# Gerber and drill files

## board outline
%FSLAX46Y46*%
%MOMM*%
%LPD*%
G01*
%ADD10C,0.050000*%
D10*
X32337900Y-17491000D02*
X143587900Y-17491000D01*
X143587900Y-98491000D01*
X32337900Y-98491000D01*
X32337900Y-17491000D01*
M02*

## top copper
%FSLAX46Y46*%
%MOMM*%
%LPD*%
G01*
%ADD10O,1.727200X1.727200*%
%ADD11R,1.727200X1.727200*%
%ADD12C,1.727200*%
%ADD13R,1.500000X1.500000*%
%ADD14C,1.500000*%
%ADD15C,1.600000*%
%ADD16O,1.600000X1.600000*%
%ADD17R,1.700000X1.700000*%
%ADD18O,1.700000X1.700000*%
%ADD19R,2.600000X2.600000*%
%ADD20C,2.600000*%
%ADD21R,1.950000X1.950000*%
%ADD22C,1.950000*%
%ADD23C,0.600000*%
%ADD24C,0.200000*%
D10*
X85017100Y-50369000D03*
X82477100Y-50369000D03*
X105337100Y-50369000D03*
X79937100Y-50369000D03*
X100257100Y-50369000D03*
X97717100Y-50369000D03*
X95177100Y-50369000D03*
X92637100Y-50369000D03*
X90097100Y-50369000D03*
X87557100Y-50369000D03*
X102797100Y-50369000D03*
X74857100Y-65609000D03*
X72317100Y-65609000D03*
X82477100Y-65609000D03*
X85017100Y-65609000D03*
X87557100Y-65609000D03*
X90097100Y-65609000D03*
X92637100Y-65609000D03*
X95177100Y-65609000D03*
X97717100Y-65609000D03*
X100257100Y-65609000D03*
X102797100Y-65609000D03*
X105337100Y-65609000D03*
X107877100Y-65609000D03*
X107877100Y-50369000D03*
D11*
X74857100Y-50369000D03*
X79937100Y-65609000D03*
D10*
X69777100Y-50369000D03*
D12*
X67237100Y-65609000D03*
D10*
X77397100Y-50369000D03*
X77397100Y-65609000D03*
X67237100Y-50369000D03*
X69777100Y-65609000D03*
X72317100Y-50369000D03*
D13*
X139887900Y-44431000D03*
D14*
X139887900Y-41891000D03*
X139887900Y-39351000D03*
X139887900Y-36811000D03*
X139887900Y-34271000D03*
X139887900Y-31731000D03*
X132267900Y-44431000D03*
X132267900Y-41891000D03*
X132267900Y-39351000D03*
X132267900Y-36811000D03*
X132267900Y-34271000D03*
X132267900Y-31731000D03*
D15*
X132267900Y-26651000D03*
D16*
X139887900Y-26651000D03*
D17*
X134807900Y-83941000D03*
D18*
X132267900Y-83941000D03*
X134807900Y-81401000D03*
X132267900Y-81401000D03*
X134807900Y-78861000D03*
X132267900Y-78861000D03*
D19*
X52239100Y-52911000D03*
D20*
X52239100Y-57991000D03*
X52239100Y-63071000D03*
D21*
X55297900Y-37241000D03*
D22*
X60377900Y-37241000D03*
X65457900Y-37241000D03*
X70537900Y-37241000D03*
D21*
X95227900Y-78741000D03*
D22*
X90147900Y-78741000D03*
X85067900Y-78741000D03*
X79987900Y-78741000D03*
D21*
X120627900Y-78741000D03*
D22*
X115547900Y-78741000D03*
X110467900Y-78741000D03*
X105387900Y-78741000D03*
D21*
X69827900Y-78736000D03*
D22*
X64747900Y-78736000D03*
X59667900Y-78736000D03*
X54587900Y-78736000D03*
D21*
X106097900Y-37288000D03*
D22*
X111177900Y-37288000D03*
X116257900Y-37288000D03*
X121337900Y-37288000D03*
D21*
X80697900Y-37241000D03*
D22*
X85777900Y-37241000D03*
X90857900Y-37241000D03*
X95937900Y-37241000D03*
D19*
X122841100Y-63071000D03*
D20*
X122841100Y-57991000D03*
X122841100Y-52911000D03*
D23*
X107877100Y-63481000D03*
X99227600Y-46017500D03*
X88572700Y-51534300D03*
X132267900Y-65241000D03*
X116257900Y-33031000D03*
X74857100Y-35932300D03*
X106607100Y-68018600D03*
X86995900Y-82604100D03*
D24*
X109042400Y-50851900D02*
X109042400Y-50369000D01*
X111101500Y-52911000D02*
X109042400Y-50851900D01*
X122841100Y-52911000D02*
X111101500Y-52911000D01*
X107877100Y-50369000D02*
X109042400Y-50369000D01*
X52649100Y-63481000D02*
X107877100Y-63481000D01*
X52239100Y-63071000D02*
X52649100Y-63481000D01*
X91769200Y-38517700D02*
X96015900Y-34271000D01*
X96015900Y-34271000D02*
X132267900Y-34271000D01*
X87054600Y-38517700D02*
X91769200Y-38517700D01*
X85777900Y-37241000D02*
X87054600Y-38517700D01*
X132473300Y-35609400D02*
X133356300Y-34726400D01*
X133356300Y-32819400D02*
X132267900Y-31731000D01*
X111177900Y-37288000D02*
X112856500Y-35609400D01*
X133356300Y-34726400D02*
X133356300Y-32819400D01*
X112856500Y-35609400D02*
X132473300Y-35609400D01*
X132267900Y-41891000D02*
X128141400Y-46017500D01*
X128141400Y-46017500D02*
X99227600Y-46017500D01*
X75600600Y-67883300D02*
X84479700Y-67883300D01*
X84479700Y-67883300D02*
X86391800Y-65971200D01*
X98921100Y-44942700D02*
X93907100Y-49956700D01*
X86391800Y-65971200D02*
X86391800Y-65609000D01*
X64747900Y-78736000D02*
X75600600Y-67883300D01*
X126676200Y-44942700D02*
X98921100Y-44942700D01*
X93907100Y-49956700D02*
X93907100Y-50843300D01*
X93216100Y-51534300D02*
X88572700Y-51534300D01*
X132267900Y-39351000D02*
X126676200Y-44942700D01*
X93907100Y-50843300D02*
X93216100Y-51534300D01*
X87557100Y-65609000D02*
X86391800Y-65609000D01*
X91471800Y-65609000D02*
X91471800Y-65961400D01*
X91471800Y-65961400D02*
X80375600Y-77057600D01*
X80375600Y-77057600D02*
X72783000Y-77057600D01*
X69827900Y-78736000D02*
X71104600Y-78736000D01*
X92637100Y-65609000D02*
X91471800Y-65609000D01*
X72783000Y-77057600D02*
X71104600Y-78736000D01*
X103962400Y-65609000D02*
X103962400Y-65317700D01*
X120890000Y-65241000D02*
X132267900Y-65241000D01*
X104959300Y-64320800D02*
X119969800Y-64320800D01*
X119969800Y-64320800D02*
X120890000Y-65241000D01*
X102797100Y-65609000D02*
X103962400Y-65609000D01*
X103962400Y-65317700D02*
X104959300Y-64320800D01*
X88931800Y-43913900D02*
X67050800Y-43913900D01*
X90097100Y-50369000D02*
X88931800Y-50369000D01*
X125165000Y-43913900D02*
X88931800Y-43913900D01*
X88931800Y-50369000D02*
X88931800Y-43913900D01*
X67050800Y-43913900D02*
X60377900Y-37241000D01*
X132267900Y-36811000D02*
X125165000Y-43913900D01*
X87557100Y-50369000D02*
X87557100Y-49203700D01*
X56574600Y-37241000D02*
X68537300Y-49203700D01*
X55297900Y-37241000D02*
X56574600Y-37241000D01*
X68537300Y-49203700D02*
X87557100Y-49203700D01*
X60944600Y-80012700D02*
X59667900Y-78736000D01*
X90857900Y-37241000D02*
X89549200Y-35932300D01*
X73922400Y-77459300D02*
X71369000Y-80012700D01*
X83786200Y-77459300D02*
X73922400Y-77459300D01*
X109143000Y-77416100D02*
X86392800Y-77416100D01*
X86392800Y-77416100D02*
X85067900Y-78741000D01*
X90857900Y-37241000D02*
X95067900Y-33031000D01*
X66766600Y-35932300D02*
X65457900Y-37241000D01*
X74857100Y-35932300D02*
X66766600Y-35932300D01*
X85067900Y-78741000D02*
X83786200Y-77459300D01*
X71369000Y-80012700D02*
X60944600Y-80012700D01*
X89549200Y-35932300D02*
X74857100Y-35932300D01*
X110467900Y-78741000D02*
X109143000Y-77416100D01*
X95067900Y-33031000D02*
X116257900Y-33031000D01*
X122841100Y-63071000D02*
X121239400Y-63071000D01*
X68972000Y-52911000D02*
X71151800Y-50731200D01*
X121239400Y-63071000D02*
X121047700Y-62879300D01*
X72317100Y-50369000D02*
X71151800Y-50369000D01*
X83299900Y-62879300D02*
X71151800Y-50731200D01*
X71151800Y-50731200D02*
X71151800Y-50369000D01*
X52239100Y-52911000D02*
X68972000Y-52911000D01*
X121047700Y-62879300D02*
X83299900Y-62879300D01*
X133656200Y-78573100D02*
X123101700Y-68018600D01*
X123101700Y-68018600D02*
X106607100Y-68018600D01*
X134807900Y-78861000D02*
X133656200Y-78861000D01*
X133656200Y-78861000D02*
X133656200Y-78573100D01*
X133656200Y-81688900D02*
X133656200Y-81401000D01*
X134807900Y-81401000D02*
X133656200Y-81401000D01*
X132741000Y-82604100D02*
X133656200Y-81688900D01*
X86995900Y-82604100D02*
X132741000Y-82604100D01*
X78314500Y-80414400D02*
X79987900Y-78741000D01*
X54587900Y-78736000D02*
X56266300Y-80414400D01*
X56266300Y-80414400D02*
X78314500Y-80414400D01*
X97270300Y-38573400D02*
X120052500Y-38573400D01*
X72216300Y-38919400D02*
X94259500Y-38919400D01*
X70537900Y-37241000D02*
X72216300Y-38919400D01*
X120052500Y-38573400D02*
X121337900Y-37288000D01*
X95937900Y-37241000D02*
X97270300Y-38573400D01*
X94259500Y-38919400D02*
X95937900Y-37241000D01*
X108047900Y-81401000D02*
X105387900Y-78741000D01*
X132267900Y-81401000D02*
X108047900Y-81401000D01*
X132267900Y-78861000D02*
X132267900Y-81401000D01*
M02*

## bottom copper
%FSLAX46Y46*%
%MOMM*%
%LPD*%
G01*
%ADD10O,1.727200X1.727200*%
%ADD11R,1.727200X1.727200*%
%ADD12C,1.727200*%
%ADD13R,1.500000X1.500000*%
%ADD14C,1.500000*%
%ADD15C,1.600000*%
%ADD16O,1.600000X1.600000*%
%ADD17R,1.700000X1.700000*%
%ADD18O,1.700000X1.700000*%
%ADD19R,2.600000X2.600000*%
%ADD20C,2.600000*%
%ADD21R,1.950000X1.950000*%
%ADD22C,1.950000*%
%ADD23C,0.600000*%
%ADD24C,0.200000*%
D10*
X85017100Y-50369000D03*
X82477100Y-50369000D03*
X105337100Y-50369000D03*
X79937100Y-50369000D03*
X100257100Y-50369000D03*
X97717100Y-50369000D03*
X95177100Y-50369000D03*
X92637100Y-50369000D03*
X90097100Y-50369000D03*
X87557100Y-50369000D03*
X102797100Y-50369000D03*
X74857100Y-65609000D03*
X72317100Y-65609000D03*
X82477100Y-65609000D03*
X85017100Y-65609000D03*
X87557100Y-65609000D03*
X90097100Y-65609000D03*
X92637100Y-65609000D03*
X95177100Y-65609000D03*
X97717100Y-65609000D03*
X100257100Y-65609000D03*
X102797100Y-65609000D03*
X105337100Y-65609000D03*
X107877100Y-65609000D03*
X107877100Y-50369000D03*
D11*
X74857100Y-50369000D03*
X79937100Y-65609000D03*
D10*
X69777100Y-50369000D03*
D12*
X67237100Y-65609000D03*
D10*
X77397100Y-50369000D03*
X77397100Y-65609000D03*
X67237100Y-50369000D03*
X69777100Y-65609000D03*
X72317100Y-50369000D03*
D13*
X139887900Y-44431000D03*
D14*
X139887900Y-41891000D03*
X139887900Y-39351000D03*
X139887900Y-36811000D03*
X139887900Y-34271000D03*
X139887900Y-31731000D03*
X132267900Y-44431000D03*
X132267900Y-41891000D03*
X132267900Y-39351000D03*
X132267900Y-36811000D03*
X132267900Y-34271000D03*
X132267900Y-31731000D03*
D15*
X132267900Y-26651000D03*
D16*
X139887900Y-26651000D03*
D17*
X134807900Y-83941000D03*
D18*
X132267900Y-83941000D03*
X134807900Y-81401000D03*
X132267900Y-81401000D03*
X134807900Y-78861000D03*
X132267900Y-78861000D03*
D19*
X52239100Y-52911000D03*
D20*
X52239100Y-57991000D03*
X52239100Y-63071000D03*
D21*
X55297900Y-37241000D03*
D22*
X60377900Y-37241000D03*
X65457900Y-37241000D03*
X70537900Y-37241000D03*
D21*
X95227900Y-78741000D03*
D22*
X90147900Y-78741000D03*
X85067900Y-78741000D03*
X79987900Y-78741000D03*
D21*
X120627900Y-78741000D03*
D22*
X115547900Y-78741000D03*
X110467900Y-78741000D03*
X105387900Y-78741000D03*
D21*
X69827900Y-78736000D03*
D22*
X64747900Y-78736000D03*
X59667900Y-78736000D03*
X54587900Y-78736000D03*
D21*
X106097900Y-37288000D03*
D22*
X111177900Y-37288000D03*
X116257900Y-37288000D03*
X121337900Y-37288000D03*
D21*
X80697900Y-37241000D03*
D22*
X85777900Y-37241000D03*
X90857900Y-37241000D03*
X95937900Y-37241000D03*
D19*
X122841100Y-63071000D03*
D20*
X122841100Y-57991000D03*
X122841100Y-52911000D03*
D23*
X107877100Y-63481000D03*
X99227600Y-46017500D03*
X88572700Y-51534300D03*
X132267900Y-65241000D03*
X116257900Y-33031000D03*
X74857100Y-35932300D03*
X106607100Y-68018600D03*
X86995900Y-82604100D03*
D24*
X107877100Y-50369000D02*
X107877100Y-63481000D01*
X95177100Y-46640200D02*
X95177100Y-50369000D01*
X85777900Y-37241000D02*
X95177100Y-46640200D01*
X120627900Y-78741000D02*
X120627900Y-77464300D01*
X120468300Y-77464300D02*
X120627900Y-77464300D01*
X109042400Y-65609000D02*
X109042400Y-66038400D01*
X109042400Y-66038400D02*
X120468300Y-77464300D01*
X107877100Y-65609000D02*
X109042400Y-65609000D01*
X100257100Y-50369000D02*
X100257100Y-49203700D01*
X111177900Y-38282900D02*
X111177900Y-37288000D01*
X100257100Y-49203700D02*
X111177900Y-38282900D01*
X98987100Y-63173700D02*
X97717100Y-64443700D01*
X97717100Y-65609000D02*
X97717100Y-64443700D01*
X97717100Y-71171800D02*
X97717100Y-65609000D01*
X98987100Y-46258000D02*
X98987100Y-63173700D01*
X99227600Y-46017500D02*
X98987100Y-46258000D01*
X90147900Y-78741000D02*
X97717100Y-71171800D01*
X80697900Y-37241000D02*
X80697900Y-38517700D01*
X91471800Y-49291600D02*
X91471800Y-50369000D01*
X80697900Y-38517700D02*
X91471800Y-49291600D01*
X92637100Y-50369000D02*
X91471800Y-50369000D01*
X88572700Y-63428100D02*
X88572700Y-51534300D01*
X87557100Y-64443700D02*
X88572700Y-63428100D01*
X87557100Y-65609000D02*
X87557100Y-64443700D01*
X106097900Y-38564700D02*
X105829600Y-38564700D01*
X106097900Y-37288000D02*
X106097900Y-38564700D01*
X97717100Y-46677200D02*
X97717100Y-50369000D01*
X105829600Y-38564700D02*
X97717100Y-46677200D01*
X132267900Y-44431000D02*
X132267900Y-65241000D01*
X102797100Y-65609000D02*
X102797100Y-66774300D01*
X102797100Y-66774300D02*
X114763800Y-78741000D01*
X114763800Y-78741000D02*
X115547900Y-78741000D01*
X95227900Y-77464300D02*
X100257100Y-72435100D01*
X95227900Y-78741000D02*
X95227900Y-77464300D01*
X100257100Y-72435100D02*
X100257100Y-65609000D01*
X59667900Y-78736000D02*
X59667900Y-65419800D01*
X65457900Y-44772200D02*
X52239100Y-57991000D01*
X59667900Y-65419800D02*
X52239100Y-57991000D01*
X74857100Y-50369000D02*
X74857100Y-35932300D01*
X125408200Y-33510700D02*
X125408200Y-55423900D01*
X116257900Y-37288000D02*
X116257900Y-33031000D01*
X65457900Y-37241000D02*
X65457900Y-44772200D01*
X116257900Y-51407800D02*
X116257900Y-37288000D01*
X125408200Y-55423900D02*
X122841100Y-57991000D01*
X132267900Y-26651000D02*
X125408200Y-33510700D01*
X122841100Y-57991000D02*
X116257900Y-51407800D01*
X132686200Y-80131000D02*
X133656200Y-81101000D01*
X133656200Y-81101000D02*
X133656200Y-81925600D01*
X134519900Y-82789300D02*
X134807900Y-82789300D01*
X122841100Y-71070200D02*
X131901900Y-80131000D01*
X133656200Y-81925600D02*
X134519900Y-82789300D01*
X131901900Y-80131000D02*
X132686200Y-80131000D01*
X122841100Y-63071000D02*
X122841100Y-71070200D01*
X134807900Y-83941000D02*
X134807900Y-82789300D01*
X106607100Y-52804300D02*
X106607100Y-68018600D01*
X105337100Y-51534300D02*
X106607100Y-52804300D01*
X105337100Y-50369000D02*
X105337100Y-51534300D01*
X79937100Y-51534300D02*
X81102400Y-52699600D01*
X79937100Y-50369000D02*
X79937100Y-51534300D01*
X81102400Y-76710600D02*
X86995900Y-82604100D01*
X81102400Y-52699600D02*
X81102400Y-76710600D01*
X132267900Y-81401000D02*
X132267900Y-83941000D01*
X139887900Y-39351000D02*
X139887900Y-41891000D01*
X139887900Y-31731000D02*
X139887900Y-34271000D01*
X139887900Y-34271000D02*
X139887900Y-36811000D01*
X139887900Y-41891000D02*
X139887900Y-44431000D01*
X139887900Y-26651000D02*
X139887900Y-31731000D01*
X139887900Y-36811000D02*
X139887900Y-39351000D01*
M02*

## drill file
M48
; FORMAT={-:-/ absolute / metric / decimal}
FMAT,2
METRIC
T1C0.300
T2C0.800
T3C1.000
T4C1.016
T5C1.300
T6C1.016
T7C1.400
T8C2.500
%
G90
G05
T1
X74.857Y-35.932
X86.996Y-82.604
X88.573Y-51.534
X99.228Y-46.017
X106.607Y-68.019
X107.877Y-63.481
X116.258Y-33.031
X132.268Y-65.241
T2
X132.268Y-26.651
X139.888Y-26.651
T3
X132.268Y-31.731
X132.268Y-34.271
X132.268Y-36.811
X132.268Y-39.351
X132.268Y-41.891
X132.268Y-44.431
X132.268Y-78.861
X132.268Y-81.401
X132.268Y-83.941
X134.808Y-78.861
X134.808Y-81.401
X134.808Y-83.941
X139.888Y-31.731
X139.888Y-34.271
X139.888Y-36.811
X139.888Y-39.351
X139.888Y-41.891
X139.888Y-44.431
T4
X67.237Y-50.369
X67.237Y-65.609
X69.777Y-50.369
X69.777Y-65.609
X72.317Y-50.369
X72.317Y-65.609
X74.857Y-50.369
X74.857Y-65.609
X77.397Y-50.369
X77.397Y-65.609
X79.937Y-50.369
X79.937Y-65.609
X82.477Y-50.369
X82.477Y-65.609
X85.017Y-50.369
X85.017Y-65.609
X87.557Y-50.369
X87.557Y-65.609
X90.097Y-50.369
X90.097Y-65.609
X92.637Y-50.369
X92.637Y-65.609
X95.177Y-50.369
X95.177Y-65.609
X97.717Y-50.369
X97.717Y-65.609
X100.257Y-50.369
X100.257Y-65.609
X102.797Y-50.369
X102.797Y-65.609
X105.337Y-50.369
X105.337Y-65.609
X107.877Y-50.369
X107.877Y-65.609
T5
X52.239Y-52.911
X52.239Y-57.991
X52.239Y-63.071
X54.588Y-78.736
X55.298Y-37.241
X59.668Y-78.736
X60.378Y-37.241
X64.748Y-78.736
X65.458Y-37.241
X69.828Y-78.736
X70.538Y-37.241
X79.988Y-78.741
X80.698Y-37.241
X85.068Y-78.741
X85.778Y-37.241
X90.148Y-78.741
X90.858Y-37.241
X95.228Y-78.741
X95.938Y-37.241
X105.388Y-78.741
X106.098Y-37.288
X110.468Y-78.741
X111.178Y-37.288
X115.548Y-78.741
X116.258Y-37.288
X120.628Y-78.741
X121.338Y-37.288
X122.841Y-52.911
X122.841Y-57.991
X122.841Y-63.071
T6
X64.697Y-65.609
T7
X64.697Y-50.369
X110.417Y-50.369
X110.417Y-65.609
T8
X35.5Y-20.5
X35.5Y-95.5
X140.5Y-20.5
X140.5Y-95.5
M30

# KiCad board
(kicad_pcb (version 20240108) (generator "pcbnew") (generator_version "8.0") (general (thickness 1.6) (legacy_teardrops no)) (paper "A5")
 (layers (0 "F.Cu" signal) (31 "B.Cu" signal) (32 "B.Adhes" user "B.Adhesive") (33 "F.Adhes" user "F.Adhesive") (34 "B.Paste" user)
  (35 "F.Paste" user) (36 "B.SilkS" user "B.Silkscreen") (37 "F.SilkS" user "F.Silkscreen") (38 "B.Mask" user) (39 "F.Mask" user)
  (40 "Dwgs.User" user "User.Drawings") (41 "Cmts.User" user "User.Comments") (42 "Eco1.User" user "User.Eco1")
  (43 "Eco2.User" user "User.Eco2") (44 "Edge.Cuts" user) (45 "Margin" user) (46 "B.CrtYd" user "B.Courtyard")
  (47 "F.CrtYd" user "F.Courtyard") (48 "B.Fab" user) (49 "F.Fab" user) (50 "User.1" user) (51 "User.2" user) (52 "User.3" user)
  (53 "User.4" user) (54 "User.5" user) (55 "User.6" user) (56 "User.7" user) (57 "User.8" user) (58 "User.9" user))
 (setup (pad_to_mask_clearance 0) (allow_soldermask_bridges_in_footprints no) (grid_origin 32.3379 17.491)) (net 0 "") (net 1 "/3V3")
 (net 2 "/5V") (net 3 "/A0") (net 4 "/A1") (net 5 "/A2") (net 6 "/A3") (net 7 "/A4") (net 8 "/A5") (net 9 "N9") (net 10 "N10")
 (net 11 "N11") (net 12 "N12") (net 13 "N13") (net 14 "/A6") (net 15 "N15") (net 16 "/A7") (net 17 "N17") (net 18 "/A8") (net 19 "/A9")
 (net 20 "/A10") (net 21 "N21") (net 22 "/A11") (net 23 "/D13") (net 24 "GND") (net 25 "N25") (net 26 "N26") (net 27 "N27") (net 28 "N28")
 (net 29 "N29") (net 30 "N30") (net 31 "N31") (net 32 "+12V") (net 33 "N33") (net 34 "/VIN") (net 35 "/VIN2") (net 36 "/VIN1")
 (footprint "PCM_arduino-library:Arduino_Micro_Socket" (layer "F.Cu") (at 111.7971 48.989 180)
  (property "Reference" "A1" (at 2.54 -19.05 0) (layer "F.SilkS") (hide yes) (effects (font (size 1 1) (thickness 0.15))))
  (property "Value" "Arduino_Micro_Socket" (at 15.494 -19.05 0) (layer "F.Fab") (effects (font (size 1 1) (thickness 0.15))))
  (pad "" np_thru_hole circle (at 1.38 -16.62 180) (size 1.4 1.4) (drill 1.4) (layers "F&B.Cu" "*.Mask"))
  (pad "" np_thru_hole circle (at 1.38 -1.38 180) (size 1.4 1.4) (drill 1.4) (layers "F&B.Cu" "*.Mask"))
  (pad "" thru_hole oval (at 26.78 -1.38 180) (size 1.7272 1.7272) (drill 1.016) (layers "*.Cu" "*.Mask") (remove_unused_layers no))
  (pad "" thru_hole oval (at 29.32 -1.38 180) (size 1.7272 1.7272) (drill 1.016) (layers "*.Cu" "*.Mask") (remove_unused_layers no))
  (pad "" np_thru_hole circle (at 47.1 -16.62 180) (size 1.016 1.016) (drill 1.016) (layers "*.Cu" "*.Mask"))
  (pad "" np_thru_hole circle (at 47.1 -1.38 180) (size 1.4 1.4) (drill 1.4) (layers "F&B.Cu" "*.Mask"))
  (pad "3V3" thru_hole oval (at 6.46 -1.38 180) (size 1.7272 1.7272) (drill 1.016) (layers "*.Cu" "*.Mask") (remove_unused_layers no)
   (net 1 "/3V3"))
  (pad "5V" thru_hole oval (at 31.86 -1.38 180) (size 1.7272 1.7272) (drill 1.016) (layers "*.Cu" "*.Mask") (remove_unused_layers no)
   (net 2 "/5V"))
  (pad "A0" thru_hole oval (at 11.54 -1.38 180) (size 1.7272 1.7272) (drill 1.016) (layers "*.Cu" "*.Mask") (remove_unused_layers no)
   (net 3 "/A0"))
  (pad "A1" thru_hole oval (at 14.08 -1.38 180) (size 1.7272 1.7272) (drill 1.016) (layers "*.Cu" "*.Mask") (remove_unused_layers no)
   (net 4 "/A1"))
  (pad "A2" thru_hole oval (at 16.62 -1.38 180) (size 1.7272 1.7272) (drill 1.016) (layers "*.Cu" "*.Mask") (remove_unused_layers no)
   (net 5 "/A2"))
  (pad "A3" thru_hole oval (at 19.16 -1.38 180) (size 1.7272 1.7272) (drill 1.016) (layers "*.Cu" "*.Mask") (remove_unused_layers no)
   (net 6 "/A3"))
  (pad "A4" thru_hole oval (at 21.7 -1.38 180) (size 1.7272 1.7272) (drill 1.016) (layers "*.Cu" "*.Mask") (remove_unused_layers no)
   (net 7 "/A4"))
  (pad "A5" thru_hole oval (at 24.24 -1.38 180) (size 1.7272 1.7272) (drill 1.016) (layers "*.Cu" "*.Mask") (remove_unused_layers no)
   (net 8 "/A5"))
  (pad "AREF" thru_hole oval (at 9 -1.38 180) (size 1.7272 1.7272) (drill 1.016) (layers "*.Cu" "*.Mask") (remove_unused_layers no)
   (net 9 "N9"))
  (pad "D0" thru_hole oval (at 36.94 -16.62 180) (size 1.7272 1.7272) (drill 1.016) (layers "*.Cu" "*.Mask") (remove_unused_layers no)
   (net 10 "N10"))
  (pad "D1" thru_hole oval (at 39.48 -16.62 180) (size 1.7272 1.7272) (drill 1.016) (layers "*.Cu" "*.Mask") (remove_unused_layers no)
   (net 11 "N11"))
  (pad "D2" thru_hole oval (at 29.32 -16.62 180) (size 1.7272 1.7272) (drill 1.016) (layers "*.Cu" "*.Mask") (remove_unused_layers no)
   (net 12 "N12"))
  (pad "D3" thru_hole oval (at 26.78 -16.62 180) (size 1.7272 1.7272) (drill 1.016) (layers "*.Cu" "*.Mask") (remove_unused_layers no)
   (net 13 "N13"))
  (pad "D4" thru_hole oval (at 24.24 -16.62 180) (size 1.7272 1.7272) (drill 1.016) (layers "*.Cu" "*.Mask") (remove_unused_layers no)
   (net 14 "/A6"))
  (pad "D5" thru_hole oval (at 21.7 -16.62 180) (size 1.7272 1.7272) (drill 1.016) (layers "*.Cu" "*.Mask") (remove_unused_layers no)
   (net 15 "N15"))
  (pad "D6" thru_hole oval (at 19.16 -16.62 180) (size 1.7272 1.7272) (drill 1.016) (layers "*.Cu" "*.Mask") (remove_unused_layers no)
   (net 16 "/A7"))
  (pad "D7" thru_hole oval (at 16.62 -16.62 180) (size 1.7272 1.7272) (drill 1.016) (layers "*.Cu" "*.Mask") (remove_unused_layers no)
   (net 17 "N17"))
  (pad "D8" thru_hole oval (at 14.08 -16.62 180) (size 1.7272 1.7272) (drill 1.016) (layers "*.Cu" "*.Mask") (remove_unused_layers no)
   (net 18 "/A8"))
  (pad "D9" thru_hole oval (at 11.54 -16.62 180) (size 1.7272 1.7272) (drill 1.016) (layers "*.Cu" "*.Mask") (remove_unused_layers no)
   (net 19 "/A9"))
  (pad "D10" thru_hole oval (at 9 -16.62 180) (size 1.7272 1.7272) (drill 1.016) (layers "*.Cu" "*.Mask") (remove_unused_layers no)
   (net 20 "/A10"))
  (pad "D11" thru_hole oval (at 6.46 -16.62 180) (size 1.7272 1.7272) (drill 1.016) (layers "*.Cu" "*.Mask") (remove_unused_layers no)
   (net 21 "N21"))
  (pad "D12" thru_hole oval (at 3.92 -16.62 180) (size 1.7272 1.7272) (drill 1.016) (layers "*.Cu" "*.Mask") (remove_unused_layers no)
   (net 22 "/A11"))
  (pad "D13" thru_hole oval (at 3.92 -1.38 180) (size 1.7272 1.7272) (drill 1.016) (layers "*.Cu" "*.Mask") (remove_unused_layers no)
   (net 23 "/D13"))
  (pad "GND1" thru_hole rect (at 36.94 -1.38 180) (size 1.7272 1.7272) (drill 1.016) (layers "*.Cu" "*.Mask") (remove_unused_layers no)
   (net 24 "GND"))
  (pad "GND2" thru_hole rect (at 31.86 -16.62 180) (size 1.7272 1.7272) (drill 1.016) (layers "*.Cu" "*.Mask") (remove_unused_layers no)
   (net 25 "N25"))
  (pad "MISO" thru_hole oval (at 42.02 -1.38 180) (size 1.7272 1.7272) (drill 1.016) (layers "*.Cu" "*.Mask") (remove_unused_layers no)
   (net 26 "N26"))
  (pad "MOSI" thru_hole circle (at 44.56 -16.62 180) (size 1.7272 1.7272) (drill 1.016) (layers "*.Cu" "*.Mask") (remove_unused_layers no)
   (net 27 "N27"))
  (pad "RST1" thru_hole oval (at 34.4 -1.38 180) (size 1.7272 1.7272) (drill 1.016) (layers "*.Cu" "*.Mask") (remove_unused_layers no)
   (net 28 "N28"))
  (pad "RST2" thru_hole oval (at 34.4 -16.62 180) (size 1.7272 1.7272) (drill 1.016) (layers "*.Cu" "*.Mask") (remove_unused_layers no)
   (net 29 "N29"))
  (pad "SCK" thru_hole oval (at 44.56 -1.38 180) (size 1.7272 1.7272) (drill 1.016) (layers "*.Cu" "*.Mask") (remove_unused_layers no)
   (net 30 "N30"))
  (pad "SS" thru_hole oval (at 42.02 -16.62 180) (size 1.7272 1.7272) (drill 1.016) (layers "*.Cu" "*.Mask") (remove_unused_layers no)
   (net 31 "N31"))
  (pad "VIN" thru_hole oval (at 39.48 -1.38 180) (size 1.7272 1.7272) (drill 1.016) (layers "*.Cu" "*.Mask") (remove_unused_layers no)
   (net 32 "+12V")))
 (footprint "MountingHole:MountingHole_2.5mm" (layer "F.Cu") (at 35.5 20.5)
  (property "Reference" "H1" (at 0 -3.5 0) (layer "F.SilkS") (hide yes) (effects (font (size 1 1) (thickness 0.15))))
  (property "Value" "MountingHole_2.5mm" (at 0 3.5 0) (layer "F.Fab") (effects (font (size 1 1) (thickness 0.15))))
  (pad "" np_thru_hole circle (at 0 0) (size 2.5 2.5) (drill 2.5) (layers "*.Cu" "*.Mask")))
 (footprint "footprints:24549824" (layer "F.Cu") (at 139.8879 44.431 90)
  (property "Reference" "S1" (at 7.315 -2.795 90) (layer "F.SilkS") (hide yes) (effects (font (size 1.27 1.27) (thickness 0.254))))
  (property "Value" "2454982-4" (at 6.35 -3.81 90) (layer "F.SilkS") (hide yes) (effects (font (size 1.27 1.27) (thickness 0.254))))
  (pad "A1" thru_hole rect (at 0 0 90) (size 1.5 1.5) (drill 1) (layers "*.Cu" "*.Mask") (remove_unused_layers no) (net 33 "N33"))
  (pad "A2" thru_hole circle (at 2.54 0 90) (size 1.5 1.5) (drill 1) (layers "*.Cu" "*.Mask") (remove_unused_layers no) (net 33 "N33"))
  (pad "A3" thru_hole circle (at 5.08 0 90) (size 1.5 1.5) (drill 1) (layers "*.Cu" "*.Mask") (remove_unused_layers no) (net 33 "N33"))
  (pad "A4" thru_hole circle (at 7.62 0 90) (size 1.5 1.5) (drill 1) (layers "*.Cu" "*.Mask") (remove_unused_layers no) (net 33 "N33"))
  (pad "A5" thru_hole circle (at 10.16 0 90) (size 1.5 1.5) (drill 1) (layers "*.Cu" "*.Mask") (remove_unused_layers no) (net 33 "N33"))
  (pad "A6" thru_hole circle (at 12.7 0 90) (size 1.5 1.5) (drill 1) (layers "*.Cu" "*.Mask") (remove_unused_layers no) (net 33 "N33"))
  (pad "B1" thru_hole circle (at 0 -7.62 90) (size 1.5 1.5) (drill 1) (layers "*.Cu" "*.Mask") (remove_unused_layers no) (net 20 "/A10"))
  (pad "B2" thru_hole circle (at 2.54 -7.62 90) (size 1.5 1.5) (drill 1) (layers "*.Cu" "*.Mask") (remove_unused_layers no) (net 18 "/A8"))
  (pad "B3" thru_hole circle (at 5.08 -7.62 90) (size 1.5 1.5) (drill 1) (layers "*.Cu" "*.Mask") (remove_unused_layers no) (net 14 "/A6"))
  (pad "B4" thru_hole circle (at 7.62 -7.62 90) (size 1.5 1.5) (drill 1) (layers "*.Cu" "*.Mask") (remove_unused_layers no) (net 7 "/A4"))
  (pad "B5" thru_hole circle (at 10.16 -7.62 90) (size 1.5 1.5) (drill 1) (layers "*.Cu" "*.Mask") (remove_unused_layers no) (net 5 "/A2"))
  (pad "B6" thru_hole circle (at 12.7 -7.62 90) (size 1.5 1.5) (drill 1) (layers "*.Cu" "*.Mask") (remove_unused_layers no) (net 3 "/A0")))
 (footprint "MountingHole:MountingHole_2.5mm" (layer "F.Cu") (at 140.5 20.5)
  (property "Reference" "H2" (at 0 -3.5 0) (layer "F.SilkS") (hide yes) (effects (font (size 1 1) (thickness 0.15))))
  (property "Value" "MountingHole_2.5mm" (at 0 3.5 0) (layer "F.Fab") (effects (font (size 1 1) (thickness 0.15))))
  (pad "" np_thru_hole circle (at 0 0) (size 2.5 2.5) (drill 2.5) (layers "*.Cu" "*.Mask")))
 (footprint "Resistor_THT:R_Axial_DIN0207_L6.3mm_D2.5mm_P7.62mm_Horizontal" (layer "F.Cu") (at 132.2679 26.651)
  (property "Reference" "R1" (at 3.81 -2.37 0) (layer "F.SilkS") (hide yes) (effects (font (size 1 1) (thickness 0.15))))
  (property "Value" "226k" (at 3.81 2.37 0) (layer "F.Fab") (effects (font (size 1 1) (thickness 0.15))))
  (pad "1" thru_hole circle (at 0 0) (size 1.6 1.6) (drill 0.8) (layers "*.Cu" "*.Mask") (remove_unused_layers no) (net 24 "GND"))
  (pad "2" thru_hole oval (at 7.62 0) (size 1.6 1.6) (drill 0.8) (layers "*.Cu" "*.Mask") (remove_unused_layers no) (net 33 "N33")))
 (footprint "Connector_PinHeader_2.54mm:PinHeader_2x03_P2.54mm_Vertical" (layer "F.Cu") (at 134.8079 83.941 180)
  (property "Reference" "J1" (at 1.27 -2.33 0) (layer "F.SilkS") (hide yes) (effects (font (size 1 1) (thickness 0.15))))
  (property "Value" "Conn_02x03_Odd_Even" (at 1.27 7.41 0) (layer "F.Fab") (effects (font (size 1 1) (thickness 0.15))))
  (pad "1" thru_hole rect (at 0 0 180) (size 1.7 1.7) (drill 1) (layers "*.Cu" "*.Mask") (remove_unused_layers no) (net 32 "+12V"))
  (pad "2" thru_hole oval (at 2.54 0 180) (size 1.7 1.7) (drill 1) (layers "*.Cu" "*.Mask") (remove_unused_layers no) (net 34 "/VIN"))
  (pad "3" thru_hole oval (at 0 2.54 180) (size 1.7 1.7) (drill 1) (layers "*.Cu" "*.Mask") (remove_unused_layers no) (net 2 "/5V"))
  (pad "4" thru_hole oval (at 2.54 2.54 180) (size 1.7 1.7) (drill 1) (layers "*.Cu" "*.Mask") (remove_unused_layers no) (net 34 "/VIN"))
  (pad "5" thru_hole oval (at 0 5.08 180) (size 1.7 1.7) (drill 1) (layers "*.Cu" "*.Mask") (remove_unused_layers no) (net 1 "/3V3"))
  (pad "6" thru_hole oval (at 2.54 5.08 180) (size 1.7 1.7) (drill 1) (layers "*.Cu" "*.Mask") (remove_unused_layers no) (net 34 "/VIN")))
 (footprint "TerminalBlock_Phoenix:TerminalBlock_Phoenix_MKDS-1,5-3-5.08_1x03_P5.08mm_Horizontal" (layer "F.Cu") (at 52.2391 52.911 -90)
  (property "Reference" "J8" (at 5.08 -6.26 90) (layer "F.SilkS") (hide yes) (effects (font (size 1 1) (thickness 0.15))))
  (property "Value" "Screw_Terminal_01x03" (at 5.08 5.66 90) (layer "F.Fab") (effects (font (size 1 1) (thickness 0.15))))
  (pad "1" thru_hole rect (at 0 0 270) (size 2.6 2.6) (drill 1.3) (layers "*.Cu" "*.Mask") (remove_unused_layers no) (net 32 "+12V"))
  (pad "2" thru_hole circle (at 5.08 0 270) (size 2.6 2.6) (drill 1.3) (layers "*.Cu" "*.Mask") (remove_unused_layers no) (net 24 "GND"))
  (pad "3" thru_hole circle (at 10.16 0 270) (size 2.6 2.6) (drill 1.3) (layers "*.Cu" "*.Mask") (remove_unused_layers no) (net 23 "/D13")))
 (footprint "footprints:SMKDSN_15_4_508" (layer "F.Cu") (at 55.2979 37.241)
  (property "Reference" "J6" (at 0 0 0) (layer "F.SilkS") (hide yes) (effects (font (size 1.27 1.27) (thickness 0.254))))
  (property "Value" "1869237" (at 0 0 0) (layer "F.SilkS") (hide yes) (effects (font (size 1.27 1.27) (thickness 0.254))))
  (pad "1" thru_hole rect (at 0 0) (size 1.95 1.95) (drill 1.3) (layers "*.Cu" "*.Mask") (remove_unused_layers no) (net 8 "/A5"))
  (pad "2" thru_hole circle (at 5.08 0) (size 1.95 1.95) (drill 1.3) (layers "*.Cu" "*.Mask") (remove_unused_layers no) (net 7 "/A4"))
  (pad "3" thru_hole circle (at 10.16 0) (size 1.95 1.95) (drill 1.3) (layers "*.Cu" "*.Mask") (remove_unused_layers no) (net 24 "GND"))
  (pad "4" thru_hole circle (at 15.24 0) (size 1.95 1.95) (drill 1.3) (layers "*.Cu" "*.Mask") (remove_unused_layers no) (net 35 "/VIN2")))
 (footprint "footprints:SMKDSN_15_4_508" (layer "F.Cu") (at 95.2279 78.741 180)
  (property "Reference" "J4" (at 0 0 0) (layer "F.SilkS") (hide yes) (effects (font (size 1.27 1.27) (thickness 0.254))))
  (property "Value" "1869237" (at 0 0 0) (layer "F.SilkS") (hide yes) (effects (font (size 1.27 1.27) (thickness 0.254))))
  (pad "1" thru_hole rect (at 0 0 180) (size 1.95 1.95) (drill 1.3) (layers "*.Cu" "*.Mask") (remove_unused_layers no) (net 19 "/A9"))
  (pad "2" thru_hole circle (at 5.08 0 180) (size 1.95 1.95) (drill 1.3) (layers "*.Cu" "*.Mask") (remove_unused_layers no) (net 18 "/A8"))
  (pad "3" thru_hole circle (at 10.16 0 180) (size 1.95 1.95) (drill 1.3) (layers "*.Cu" "*.Mask") (remove_unused_layers no) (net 24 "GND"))
  (pad "4" thru_hole circle (at 15.24 0 180) (size 1.95 1.95) (drill 1.3) (layers "*.Cu" "*.Mask") (remove_unused_layers no)
   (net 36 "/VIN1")))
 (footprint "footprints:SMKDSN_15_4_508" (layer "F.Cu") (at 120.6279 78.741 180)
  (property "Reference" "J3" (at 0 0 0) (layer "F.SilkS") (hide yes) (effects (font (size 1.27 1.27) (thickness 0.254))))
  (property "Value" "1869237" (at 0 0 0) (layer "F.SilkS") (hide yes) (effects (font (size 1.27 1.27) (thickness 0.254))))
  (pad "1" thru_hole rect (at 0 0 180) (size 1.95 1.95) (drill 1.3) (layers "*.Cu" "*.Mask") (remove_unused_layers no) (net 22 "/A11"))
  (pad "2" thru_hole circle (at 5.08 0 180) (size 1.95 1.95) (drill 1.3) (layers "*.Cu" "*.Mask") (remove_unused_layers no) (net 20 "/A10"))
  (pad "3" thru_hole circle (at 10.16 0 180) (size 1.95 1.95) (drill 1.3) (layers "*.Cu" "*.Mask") (remove_unused_layers no) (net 24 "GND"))
  (pad "4" thru_hole circle (at 15.24 0 180) (size 1.95 1.95) (drill 1.3) (layers "*.Cu" "*.Mask") (remove_unused_layers no) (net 34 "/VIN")))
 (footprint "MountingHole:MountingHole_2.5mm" (layer "F.Cu") (at 140.5 95.5)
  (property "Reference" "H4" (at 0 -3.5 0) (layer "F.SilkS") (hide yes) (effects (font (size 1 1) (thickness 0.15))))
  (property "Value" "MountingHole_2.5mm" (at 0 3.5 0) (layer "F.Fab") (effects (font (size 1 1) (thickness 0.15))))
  (pad "" np_thru_hole circle (at 0 0) (size 2.5 2.5) (drill 2.5) (layers "*.Cu" "*.Mask")))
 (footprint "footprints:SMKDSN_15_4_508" (layer "F.Cu") (at 69.8279 78.736 180)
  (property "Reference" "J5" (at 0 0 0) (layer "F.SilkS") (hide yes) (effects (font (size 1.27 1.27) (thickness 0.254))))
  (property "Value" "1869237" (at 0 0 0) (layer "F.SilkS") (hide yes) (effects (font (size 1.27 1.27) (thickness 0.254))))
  (pad "1" thru_hole rect (at 0 0 180) (size 1.95 1.95) (drill 1.3) (layers "*.Cu" "*.Mask") (remove_unused_layers no) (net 16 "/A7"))
  (pad "2" thru_hole circle (at 5.08 0 180) (size 1.95 1.95) (drill 1.3) (layers "*.Cu" "*.Mask") (remove_unused_layers no) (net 14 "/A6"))
  (pad "3" thru_hole circle (at 10.16 0 180) (size 1.95 1.95) (drill 1.3) (layers "*.Cu" "*.Mask") (remove_unused_layers no) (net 24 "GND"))
  (pad "4" thru_hole circle (at 15.24 0 180) (size 1.95 1.95) (drill 1.3) (layers "*.Cu" "*.Mask") (remove_unused_layers no)
   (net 36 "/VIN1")))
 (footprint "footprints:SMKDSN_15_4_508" (layer "F.Cu") (at 106.0979 37.288)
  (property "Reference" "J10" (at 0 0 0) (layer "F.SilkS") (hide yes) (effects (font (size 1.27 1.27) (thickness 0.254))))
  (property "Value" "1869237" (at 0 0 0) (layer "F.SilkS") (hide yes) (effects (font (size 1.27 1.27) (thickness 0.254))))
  (pad "1" thru_hole rect (at 0 0) (size 1.95 1.95) (drill 1.3) (layers "*.Cu" "*.Mask") (remove_unused_layers no) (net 4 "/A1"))
  (pad "2" thru_hole circle (at 5.08 0) (size 1.95 1.95) (drill 1.3) (layers "*.Cu" "*.Mask") (remove_unused_layers no) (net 3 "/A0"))
  (pad "3" thru_hole circle (at 10.16 0) (size 1.95 1.95) (drill 1.3) (layers "*.Cu" "*.Mask") (remove_unused_layers no) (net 24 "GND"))
  (pad "4" thru_hole circle (at 15.24 0) (size 1.95 1.95) (drill 1.3) (layers "*.Cu" "*.Mask") (remove_unused_layers no) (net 35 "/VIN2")))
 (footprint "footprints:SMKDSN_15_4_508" (layer "F.Cu") (at 80.6979 37.241)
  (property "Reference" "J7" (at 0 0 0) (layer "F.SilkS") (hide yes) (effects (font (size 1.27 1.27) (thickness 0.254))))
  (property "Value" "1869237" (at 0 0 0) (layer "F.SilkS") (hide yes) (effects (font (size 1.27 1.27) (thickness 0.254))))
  (pad "1" thru_hole rect (at 0 0) (size 1.95 1.95) (drill 1.3) (layers "*.Cu" "*.Mask") (remove_unused_layers no) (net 6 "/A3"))
  (pad "2" thru_hole circle (at 5.08 0) (size 1.95 1.95) (drill 1.3) (layers "*.Cu" "*.Mask") (remove_unused_layers no) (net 5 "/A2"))
  (pad "3" thru_hole circle (at 10.16 0) (size 1.95 1.95) (drill 1.3) (layers "*.Cu" "*.Mask") (remove_unused_layers no) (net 24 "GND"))
  (pad "4" thru_hole circle (at 15.24 0) (size 1.95 1.95) (drill 1.3) (layers "*.Cu" "*.Mask") (remove_unused_layers no) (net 35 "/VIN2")))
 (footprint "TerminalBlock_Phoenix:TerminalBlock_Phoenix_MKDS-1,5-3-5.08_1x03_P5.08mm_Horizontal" (layer "F.Cu") (at 122.8411 63.071 90)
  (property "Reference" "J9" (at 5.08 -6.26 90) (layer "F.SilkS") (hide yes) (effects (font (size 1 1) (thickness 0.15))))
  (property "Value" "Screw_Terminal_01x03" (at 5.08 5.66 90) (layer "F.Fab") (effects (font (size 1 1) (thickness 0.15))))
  (pad "1" thru_hole rect (at 0 0 90) (size 2.6 2.6) (drill 1.3) (layers "*.Cu" "*.Mask") (remove_unused_layers no) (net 32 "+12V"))
  (pad "2" thru_hole circle (at 5.08 0 90) (size 2.6 2.6) (drill 1.3) (layers "*.Cu" "*.Mask") (remove_unused_layers no) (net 24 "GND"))
  (pad "3" thru_hole circle (at 10.16 0 90) (size 2.6 2.6) (drill 1.3) (layers "*.Cu" "*.Mask") (remove_unused_layers no) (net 23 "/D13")))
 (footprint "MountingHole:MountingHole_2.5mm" (layer "F.Cu") (at 35.5 95.5)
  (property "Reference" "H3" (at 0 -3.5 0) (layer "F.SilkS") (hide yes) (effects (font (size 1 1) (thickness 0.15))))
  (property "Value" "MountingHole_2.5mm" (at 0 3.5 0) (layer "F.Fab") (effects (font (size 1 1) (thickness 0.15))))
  (pad "" np_thru_hole circle (at 0 0) (size 2.5 2.5) (drill 2.5) (layers "*.Cu" "*.Mask")))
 (gr_rect (start 32.3379 17.491) (end 143.5879 98.491) (stroke (width 0.05) (type default)) (fill none) (layer "Edge.Cuts"))
 (segment (start 109.0424 50.8519) (end 109.0424 50.369) (width 0.2) (layer "F.Cu") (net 23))
 (segment (start 111.1015 52.911) (end 109.0424 50.8519) (width 0.2) (layer "F.Cu") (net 23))
 (segment (start 122.8411 52.911) (end 111.1015 52.911) (width 0.2) (layer "F.Cu") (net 23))
 (segment (start 107.8771 50.369) (end 109.0424 50.369) (width 0.2) (layer "F.Cu") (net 23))
 (segment (start 52.6491 63.481) (end 107.8771 63.481) (width 0.2) (layer "F.Cu") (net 23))
 (segment (start 52.2391 63.071) (end 52.6491 63.481) (width 0.2) (layer "F.Cu") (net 23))
 (via (at 107.8771 63.481) (size 0.6) (drill 0.3) (layers "F.Cu" "B.Cu") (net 23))
 (segment (start 107.8771 50.369) (end 107.8771 63.481) (width 0.2) (layer "B.Cu") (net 23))
 (segment (start 91.7692 38.5177) (end 96.0159 34.271) (width 0.2) (layer "F.Cu") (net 5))
 (segment (start 96.0159 34.271) (end 132.2679 34.271) (width 0.2) (layer "F.Cu") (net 5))
 (segment (start 87.0546 38.5177) (end 91.7692 38.5177) (width 0.2) (layer "F.Cu") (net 5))
 (segment (start 85.7779 37.241) (end 87.0546 38.5177) (width 0.2) (layer "F.Cu") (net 5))
 (segment (start 95.1771 46.6402) (end 95.1771 50.369) (width 0.2) (layer "B.Cu") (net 5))
 (segment (start 85.7779 37.241) (end 95.1771 46.6402) (width 0.2) (layer "B.Cu") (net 5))
 (segment (start 120.6279 78.741) (end 120.6279 77.4643) (width 0.2) (layer "B.Cu") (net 22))
 (segment (start 120.4683 77.4643) (end 120.6279 77.4643) (width 0.2) (layer "B.Cu") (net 22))
 (segment (start 109.0424 65.609) (end 109.0424 66.0384) (width 0.2) (layer "B.Cu") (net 22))
 (segment (start 109.0424 66.0384) (end 120.4683 77.4643) (width 0.2) (layer "B.Cu") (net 22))
 (segment (start 107.8771 65.609) (end 109.0424 65.609) (width 0.2) (layer "B.Cu") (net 22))
 (segment (start 132.4733 35.6094) (end 133.3563 34.7264) (width 0.2) (layer "F.Cu") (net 3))
 (segment (start 133.3563 32.8194) (end 132.2679 31.731) (width 0.2) (layer "F.Cu") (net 3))
 (segment (start 111.1779 37.288) (end 112.8565 35.6094) (width 0.2) (layer "F.Cu") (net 3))
 (segment (start 133.3563 34.7264) (end 133.3563 32.8194) (width 0.2) (layer "F.Cu") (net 3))
 (segment (start 112.8565 35.6094) (end 132.4733 35.6094) (width 0.2) (layer "F.Cu") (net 3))
 (segment (start 100.2571 50.369) (end 100.2571 49.2037) (width 0.2) (layer "B.Cu") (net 3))
 (segment (start 111.1779 38.2829) (end 111.1779 37.288) (width 0.2) (layer "B.Cu") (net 3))
 (segment (start 100.2571 49.2037) (end 111.1779 38.2829) (width 0.2) (layer "B.Cu") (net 3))
 (segment (start 132.2679 41.891) (end 128.1414 46.0175) (width 0.2) (layer "F.Cu") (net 18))
 (segment (start 128.1414 46.0175) (end 99.2276 46.0175) (width 0.2) (layer "F.Cu") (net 18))
 (via (at 99.2276 46.0175) (size 0.6) (drill 0.3) (layers "F.Cu" "B.Cu") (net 18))
 (segment (start 98.9871 63.1737) (end 97.7171 64.4437) (width 0.2) (layer "B.Cu") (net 18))
 (segment (start 97.7171 65.609) (end 97.7171 64.4437) (width 0.2) (layer "B.Cu") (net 18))
 (segment (start 97.7171 71.1718) (end 97.7171 65.609) (width 0.2) (layer "B.Cu") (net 18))
 (segment (start 98.9871 46.258) (end 98.9871 63.1737) (width 0.2) (layer "B.Cu") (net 18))
 (segment (start 99.2276 46.0175) (end 98.9871 46.258) (width 0.2) (layer "B.Cu") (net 18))
 (segment (start 90.1479 78.741) (end 97.7171 71.1718) (width 0.2) (layer "B.Cu") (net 18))
 (segment (start 80.6979 37.241) (end 80.6979 38.5177) (width 0.2) (layer "B.Cu") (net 6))
 (segment (start 91.4718 49.2916) (end 91.4718 50.369) (width 0.2) (layer "B.Cu") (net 6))
 (segment (start 80.6979 38.5177) (end 91.4718 49.2916) (width 0.2) (layer "B.Cu") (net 6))
 (segment (start 92.6371 50.369) (end 91.4718 50.369) (width 0.2) (layer "B.Cu") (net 6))
 (segment (start 75.6006 67.8833) (end 84.4797 67.8833) (width 0.2) (layer "F.Cu") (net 14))
 (segment (start 84.4797 67.8833) (end 86.3918 65.9712) (width 0.2) (layer "F.Cu") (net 14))
 (segment (start 98.9211 44.9427) (end 93.9071 49.9567) (width 0.2) (layer "F.Cu") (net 14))
 (segment (start 86.3918 65.9712) (end 86.3918 65.609) (width 0.2) (layer "F.Cu") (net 14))
 (segment (start 64.7479 78.736) (end 75.6006 67.8833) (width 0.2) (layer "F.Cu") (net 14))
 (segment (start 126.6762 44.9427) (end 98.9211 44.9427) (width 0.2) (layer "F.Cu") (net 14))
 (segment (start 93.9071 49.9567) (end 93.9071 50.8433) (width 0.2) (layer "F.Cu") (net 14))
 (segment (start 93.2161 51.5343) (end 88.5727 51.5343) (width 0.2) (layer "F.Cu") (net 14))
 (segment (start 132.2679 39.351) (end 126.6762 44.9427) (width 0.2) (layer "F.Cu") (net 14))
 (segment (start 93.9071 50.8433) (end 93.2161 51.5343) (width 0.2) (layer "F.Cu") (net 14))
 (segment (start 87.5571 65.609) (end 86.3918 65.609) (width 0.2) (layer "F.Cu") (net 14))
 (via (at 88.5727 51.5343) (size 0.6) (drill 0.3) (layers "F.Cu" "B.Cu") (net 14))
 (segment (start 88.5727 63.4281) (end 88.5727 51.5343) (width 0.2) (layer "B.Cu") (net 14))
 (segment (start 87.5571 64.4437) (end 88.5727 63.4281) (width 0.2) (layer "B.Cu") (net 14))
 (segment (start 87.5571 65.609) (end 87.5571 64.4437) (width 0.2) (layer "B.Cu") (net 14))
 (segment (start 106.0979 38.5647) (end 105.8296 38.5647) (width 0.2) (layer "B.Cu") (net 4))
 (segment (start 106.0979 37.288) (end 106.0979 38.5647) (width 0.2) (layer "B.Cu") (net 4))
 (segment (start 97.7171 46.6772) (end 97.7171 50.369) (width 0.2) (layer "B.Cu") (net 4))
 (segment (start 105.8296 38.5647) (end 97.7171 46.6772) (width 0.2) (layer "B.Cu") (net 4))
 (segment (start 91.4718 65.609) (end 91.4718 65.9614) (width 0.2) (layer "F.Cu") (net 16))
 (segment (start 91.4718 65.9614) (end 80.3756 77.0576) (width 0.2) (layer "F.Cu") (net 16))
 (segment (start 80.3756 77.0576) (end 72.783 77.0576) (width 0.2) (layer "F.Cu") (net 16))
 (segment (start 69.8279 78.736) (end 71.1046 78.736) (width 0.2) (layer "F.Cu") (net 16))
 (segment (start 92.6371 65.609) (end 91.4718 65.609) (width 0.2) (layer "F.Cu") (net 16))
 (segment (start 72.783 77.0576) (end 71.1046 78.736) (width 0.2) (layer "F.Cu") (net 16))
 (segment (start 103.9624 65.609) (end 103.9624 65.3177) (width 0.2) (layer "F.Cu") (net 20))
 (segment (start 120.89 65.241) (end 132.2679 65.241) (width 0.2) (layer "F.Cu") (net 20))
 (segment (start 104.9593 64.3208) (end 119.9698 64.3208) (width 0.2) (layer "F.Cu") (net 20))
 (segment (start 119.9698 64.3208) (end 120.89 65.241) (width 0.2) (layer "F.Cu") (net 20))
 (segment (start 102.7971 65.609) (end 103.9624 65.609) (width 0.2) (layer "F.Cu") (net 20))
 (segment (start 103.9624 65.3177) (end 104.9593 64.3208) (width 0.2) (layer "F.Cu") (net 20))
 (via (at 132.2679 65.241) (size 0.6) (drill 0.3) (layers "F.Cu" "B.Cu") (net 20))
 (segment (start 132.2679 44.431) (end 132.2679 65.241) (width 0.2) (layer "B.Cu") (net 20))
 (segment (start 102.7971 65.609) (end 102.7971 66.7743) (width 0.2) (layer "B.Cu") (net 20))
 (segment (start 102.7971 66.7743) (end 114.7638 78.741) (width 0.2) (layer "B.Cu") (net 20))
 (segment (start 114.7638 78.741) (end 115.5479 78.741) (width 0.2) (layer "B.Cu") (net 20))
 (segment (start 88.9318 43.9139) (end 67.0508 43.9139) (width 0.2) (layer "F.Cu") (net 7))
 (segment (start 90.0971 50.369) (end 88.9318 50.369) (width 0.2) (layer "F.Cu") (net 7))
 (segment (start 125.165 43.9139) (end 88.9318 43.9139) (width 0.2) (layer "F.Cu") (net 7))
 (segment (start 88.9318 50.369) (end 88.9318 43.9139) (width 0.2) (layer "F.Cu") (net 7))
 (segment (start 67.0508 43.9139) (end 60.3779 37.241) (width 0.2) (layer "F.Cu") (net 7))
 (segment (start 132.2679 36.811) (end 125.165 43.9139) (width 0.2) (layer "F.Cu") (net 7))
 (segment (start 95.2279 77.4643) (end 100.2571 72.4351) (width 0.2) (layer "B.Cu") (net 19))
 (segment (start 95.2279 78.741) (end 95.2279 77.4643) (width 0.2) (layer "B.Cu") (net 19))
 (segment (start 100.2571 72.4351) (end 100.2571 65.609) (width 0.2) (layer "B.Cu") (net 19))
 (segment (start 87.5571 50.369) (end 87.5571 49.2037) (width 0.2) (layer "F.Cu") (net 8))
 (segment (start 56.5746 37.241) (end 68.5373 49.2037) (width 0.2) (layer "F.Cu") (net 8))
 (segment (start 55.2979 37.241) (end 56.5746 37.241) (width 0.2) (layer "F.Cu") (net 8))
 (segment (start 68.5373 49.2037) (end 87.5571 49.2037) (width 0.2) (layer "F.Cu") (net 8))
 (segment (start 60.9446 80.0127) (end 59.6679 78.736) (width 0.2) (layer "F.Cu") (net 24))
 (segment (start 90.8579 37.241) (end 89.5492 35.9323) (width 0.2) (layer "F.Cu") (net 24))
 (segment (start 73.9224 77.4593) (end 71.369 80.0127) (width 0.2) (layer "F.Cu") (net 24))
 (segment (start 83.7862 77.4593) (end 73.9224 77.4593) (width 0.2) (layer "F.Cu") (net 24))
 (segment (start 109.143 77.4161) (end 86.3928 77.4161) (width 0.2) (layer "F.Cu") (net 24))
 (segment (start 86.3928 77.4161) (end 85.0679 78.741) (width 0.2) (layer "F.Cu") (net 24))
 (segment (start 90.8579 37.241) (end 95.0679 33.031) (width 0.2) (layer "F.Cu") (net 24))
 (segment (start 66.7666 35.9323) (end 65.4579 37.241) (width 0.2) (layer "F.Cu") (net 24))
 (segment (start 74.8571 35.9323) (end 66.7666 35.9323) (width 0.2) (layer "F.Cu") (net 24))
 (segment (start 85.0679 78.741) (end 83.7862 77.4593) (width 0.2) (layer "F.Cu") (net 24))
 (segment (start 71.369 80.0127) (end 60.9446 80.0127) (width 0.2) (layer "F.Cu") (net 24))
 (segment (start 89.5492 35.9323) (end 74.8571 35.9323) (width 0.2) (layer "F.Cu") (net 24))
 (segment (start 110.4679 78.741) (end 109.143 77.4161) (width 0.2) (layer "F.Cu") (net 24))
 (segment (start 95.0679 33.031) (end 116.2579 33.031) (width 0.2) (layer "F.Cu") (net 24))
 (via (at 116.2579 33.031) (size 0.6) (drill 0.3) (layers "F.Cu" "B.Cu") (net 24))
 (via (at 74.8571 35.9323) (size 0.6) (drill 0.3) (layers "F.Cu" "B.Cu") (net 24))
 (segment (start 59.6679 78.736) (end 59.6679 65.4198) (width 0.2) (layer "B.Cu") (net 24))
 (segment (start 65.4579 44.7722) (end 52.2391 57.991) (width 0.2) (layer "B.Cu") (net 24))
 (segment (start 59.6679 65.4198) (end 52.2391 57.991) (width 0.2) (layer "B.Cu") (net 24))
 (segment (start 74.8571 50.369) (end 74.8571 35.9323) (width 0.2) (layer "B.Cu") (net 24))
 (segment (start 125.4082 33.5107) (end 125.4082 55.4239) (width 0.2) (layer "B.Cu") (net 24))
 (segment (start 116.2579 37.288) (end 116.2579 33.031) (width 0.2) (layer "B.Cu") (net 24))
 (segment (start 65.4579 37.241) (end 65.4579 44.7722) (width 0.2) (layer "B.Cu") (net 24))
 (segment (start 116.2579 51.4078) (end 116.2579 37.288) (width 0.2) (layer "B.Cu") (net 24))
 (segment (start 125.4082 55.4239) (end 122.8411 57.991) (width 0.2) (layer "B.Cu") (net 24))
 (segment (start 132.2679 26.651) (end 125.4082 33.5107) (width 0.2) (layer "B.Cu") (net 24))
 (segment (start 122.8411 57.991) (end 116.2579 51.4078) (width 0.2) (layer "B.Cu") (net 24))
 (segment (start 122.8411 63.071) (end 121.2394 63.071) (width 0.2) (layer "F.Cu") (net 32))
 (segment (start 68.972 52.911) (end 71.1518 50.7312) (width 0.2) (layer "F.Cu") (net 32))
 (segment (start 121.2394 63.071) (end 121.0477 62.8793) (width 0.2) (layer "F.Cu") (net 32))
 (segment (start 72.3171 50.369) (end 71.1518 50.369) (width 0.2) (layer "F.Cu") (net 32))
 (segment (start 83.2999 62.8793) (end 71.1518 50.7312) (width 0.2) (layer "F.Cu") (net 32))
 (segment (start 71.1518 50.7312) (end 71.1518 50.369) (width 0.2) (layer "F.Cu") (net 32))
 (segment (start 52.2391 52.911) (end 68.972 52.911) (width 0.2) (layer "F.Cu") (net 32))
 (segment (start 121.0477 62.8793) (end 83.2999 62.8793) (width 0.2) (layer "F.Cu") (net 32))
 (segment (start 132.6862 80.131) (end 133.6562 81.101) (width 0.2) (layer "B.Cu") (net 32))
 (segment (start 133.6562 81.101) (end 133.6562 81.9256) (width 0.2) (layer "B.Cu") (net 32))
 (segment (start 134.5199 82.7893) (end 134.8079 82.7893) (width 0.2) (layer "B.Cu") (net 32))
 (segment (start 122.8411 71.0702) (end 131.9019 80.131) (width 0.2) (layer "B.Cu") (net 32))
 (segment (start 133.6562 81.9256) (end 134.5199 82.7893) (width 0.2) (layer "B.Cu") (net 32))
 (segment (start 131.9019 80.131) (end 132.6862 80.131) (width 0.2) (layer "B.Cu") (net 32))
 (segment (start 122.8411 63.071) (end 122.8411 71.0702) (width 0.2) (layer "B.Cu") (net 32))
 (segment (start 134.8079 83.941) (end 134.8079 82.7893) (width 0.2) (layer "B.Cu") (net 32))
 (segment (start 133.6562 78.5731) (end 123.1017 68.0186) (width 0.2) (layer "F.Cu") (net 1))
 (segment (start 123.1017 68.0186) (end 106.6071 68.0186) (width 0.2) (layer "F.Cu") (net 1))
 (segment (start 134.8079 78.861) (end 133.6562 78.861) (width 0.2) (layer "F.Cu") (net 1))
 (segment (start 133.6562 78.861) (end 133.6562 78.5731) (width 0.2) (layer "F.Cu") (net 1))
 (via (at 106.6071 68.0186) (size 0.6) (drill 0.3) (layers "F.Cu" "B.Cu") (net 1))
 (segment (start 106.6071 52.8043) (end 106.6071 68.0186) (width 0.2) (layer "B.Cu") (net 1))
 (segment (start 105.3371 51.5343) (end 106.6071 52.8043) (width 0.2) (layer "B.Cu") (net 1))
 (segment (start 105.3371 50.369) (end 105.3371 51.5343) (width 0.2) (layer "B.Cu") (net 1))
 (segment (start 133.6562 81.6889) (end 133.6562 81.401) (width 0.2) (layer "F.Cu") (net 2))
 (segment (start 134.8079 81.401) (end 133.6562 81.401) (width 0.2) (layer "F.Cu") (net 2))
 (segment (start 132.741 82.6041) (end 133.6562 81.6889) (width 0.2) (layer "F.Cu") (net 2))
 (segment (start 86.9959 82.6041) (end 132.741 82.6041) (width 0.2) (layer "F.Cu") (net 2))
 (via (at 86.9959 82.6041) (size 0.6) (drill 0.3) (layers "F.Cu" "B.Cu") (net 2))
 (segment (start 79.9371 51.5343) (end 81.1024 52.6996) (width 0.2) (layer "B.Cu") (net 2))
 (segment (start 79.9371 50.369) (end 79.9371 51.5343) (width 0.2) (layer "B.Cu") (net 2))
 (segment (start 81.1024 76.7106) (end 86.9959 82.6041) (width 0.2) (layer "B.Cu") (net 2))
 (segment (start 81.1024 52.6996) (end 81.1024 76.7106) (width 0.2) (layer "B.Cu") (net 2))
 (segment (start 78.3145 80.4144) (end 79.9879 78.741) (width 0.2) (layer "F.Cu") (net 36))
 (segment (start 54.5879 78.736) (end 56.2663 80.4144) (width 0.2) (layer "F.Cu") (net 36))
 (segment (start 56.2663 80.4144) (end 78.3145 80.4144) (width 0.2) (layer "F.Cu") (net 36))
 (segment (start 97.2703 38.5734) (end 120.0525 38.5734) (width 0.2) (layer "F.Cu") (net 35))
 (segment (start 72.2163 38.9194) (end 94.2595 38.9194) (width 0.2) (layer "F.Cu") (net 35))
 (segment (start 70.5379 37.241) (end 72.2163 38.9194) (width 0.2) (layer "F.Cu") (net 35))
 (segment (start 120.0525 38.5734) (end 121.3379 37.288) (width 0.2) (layer "F.Cu") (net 35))
 (segment (start 95.9379 37.241) (end 97.2703 38.5734) (width 0.2) (layer "F.Cu") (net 35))
 (segment (start 94.2595 38.9194) (end 95.9379 37.241) (width 0.2) (layer "F.Cu") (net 35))
 (segment (start 108.0479 81.401) (end 105.3879 78.741) (width 0.2) (layer "F.Cu") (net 34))
 (segment (start 132.2679 81.401) (end 108.0479 81.401) (width 0.2) (layer "F.Cu") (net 34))
 (segment (start 132.2679 78.861) (end 132.2679 81.401) (width 0.2) (layer "F.Cu") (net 34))
 (segment (start 132.2679 81.401) (end 132.2679 83.941) (width 0.2) (layer "B.Cu") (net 34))
 (segment (start 139.8879 39.351) (end 139.8879 41.891) (width 0.2) (layer "B.Cu") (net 33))
 (segment (start 139.8879 31.731) (end 139.8879 34.271) (width 0.2) (layer "B.Cu") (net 33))
 (segment (start 139.8879 34.271) (end 139.8879 36.811) (width 0.2) (layer "B.Cu") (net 33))
 (segment (start 139.8879 41.891) (end 139.8879 44.431) (width 0.2) (layer "B.Cu") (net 33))
 (segment (start 139.8879 26.651) (end 139.8879 31.731) (width 0.2) (layer "B.Cu") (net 33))
 (segment (start 139.8879 36.811) (end 139.8879 39.351) (width 0.2) (layer "B.Cu") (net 33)))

